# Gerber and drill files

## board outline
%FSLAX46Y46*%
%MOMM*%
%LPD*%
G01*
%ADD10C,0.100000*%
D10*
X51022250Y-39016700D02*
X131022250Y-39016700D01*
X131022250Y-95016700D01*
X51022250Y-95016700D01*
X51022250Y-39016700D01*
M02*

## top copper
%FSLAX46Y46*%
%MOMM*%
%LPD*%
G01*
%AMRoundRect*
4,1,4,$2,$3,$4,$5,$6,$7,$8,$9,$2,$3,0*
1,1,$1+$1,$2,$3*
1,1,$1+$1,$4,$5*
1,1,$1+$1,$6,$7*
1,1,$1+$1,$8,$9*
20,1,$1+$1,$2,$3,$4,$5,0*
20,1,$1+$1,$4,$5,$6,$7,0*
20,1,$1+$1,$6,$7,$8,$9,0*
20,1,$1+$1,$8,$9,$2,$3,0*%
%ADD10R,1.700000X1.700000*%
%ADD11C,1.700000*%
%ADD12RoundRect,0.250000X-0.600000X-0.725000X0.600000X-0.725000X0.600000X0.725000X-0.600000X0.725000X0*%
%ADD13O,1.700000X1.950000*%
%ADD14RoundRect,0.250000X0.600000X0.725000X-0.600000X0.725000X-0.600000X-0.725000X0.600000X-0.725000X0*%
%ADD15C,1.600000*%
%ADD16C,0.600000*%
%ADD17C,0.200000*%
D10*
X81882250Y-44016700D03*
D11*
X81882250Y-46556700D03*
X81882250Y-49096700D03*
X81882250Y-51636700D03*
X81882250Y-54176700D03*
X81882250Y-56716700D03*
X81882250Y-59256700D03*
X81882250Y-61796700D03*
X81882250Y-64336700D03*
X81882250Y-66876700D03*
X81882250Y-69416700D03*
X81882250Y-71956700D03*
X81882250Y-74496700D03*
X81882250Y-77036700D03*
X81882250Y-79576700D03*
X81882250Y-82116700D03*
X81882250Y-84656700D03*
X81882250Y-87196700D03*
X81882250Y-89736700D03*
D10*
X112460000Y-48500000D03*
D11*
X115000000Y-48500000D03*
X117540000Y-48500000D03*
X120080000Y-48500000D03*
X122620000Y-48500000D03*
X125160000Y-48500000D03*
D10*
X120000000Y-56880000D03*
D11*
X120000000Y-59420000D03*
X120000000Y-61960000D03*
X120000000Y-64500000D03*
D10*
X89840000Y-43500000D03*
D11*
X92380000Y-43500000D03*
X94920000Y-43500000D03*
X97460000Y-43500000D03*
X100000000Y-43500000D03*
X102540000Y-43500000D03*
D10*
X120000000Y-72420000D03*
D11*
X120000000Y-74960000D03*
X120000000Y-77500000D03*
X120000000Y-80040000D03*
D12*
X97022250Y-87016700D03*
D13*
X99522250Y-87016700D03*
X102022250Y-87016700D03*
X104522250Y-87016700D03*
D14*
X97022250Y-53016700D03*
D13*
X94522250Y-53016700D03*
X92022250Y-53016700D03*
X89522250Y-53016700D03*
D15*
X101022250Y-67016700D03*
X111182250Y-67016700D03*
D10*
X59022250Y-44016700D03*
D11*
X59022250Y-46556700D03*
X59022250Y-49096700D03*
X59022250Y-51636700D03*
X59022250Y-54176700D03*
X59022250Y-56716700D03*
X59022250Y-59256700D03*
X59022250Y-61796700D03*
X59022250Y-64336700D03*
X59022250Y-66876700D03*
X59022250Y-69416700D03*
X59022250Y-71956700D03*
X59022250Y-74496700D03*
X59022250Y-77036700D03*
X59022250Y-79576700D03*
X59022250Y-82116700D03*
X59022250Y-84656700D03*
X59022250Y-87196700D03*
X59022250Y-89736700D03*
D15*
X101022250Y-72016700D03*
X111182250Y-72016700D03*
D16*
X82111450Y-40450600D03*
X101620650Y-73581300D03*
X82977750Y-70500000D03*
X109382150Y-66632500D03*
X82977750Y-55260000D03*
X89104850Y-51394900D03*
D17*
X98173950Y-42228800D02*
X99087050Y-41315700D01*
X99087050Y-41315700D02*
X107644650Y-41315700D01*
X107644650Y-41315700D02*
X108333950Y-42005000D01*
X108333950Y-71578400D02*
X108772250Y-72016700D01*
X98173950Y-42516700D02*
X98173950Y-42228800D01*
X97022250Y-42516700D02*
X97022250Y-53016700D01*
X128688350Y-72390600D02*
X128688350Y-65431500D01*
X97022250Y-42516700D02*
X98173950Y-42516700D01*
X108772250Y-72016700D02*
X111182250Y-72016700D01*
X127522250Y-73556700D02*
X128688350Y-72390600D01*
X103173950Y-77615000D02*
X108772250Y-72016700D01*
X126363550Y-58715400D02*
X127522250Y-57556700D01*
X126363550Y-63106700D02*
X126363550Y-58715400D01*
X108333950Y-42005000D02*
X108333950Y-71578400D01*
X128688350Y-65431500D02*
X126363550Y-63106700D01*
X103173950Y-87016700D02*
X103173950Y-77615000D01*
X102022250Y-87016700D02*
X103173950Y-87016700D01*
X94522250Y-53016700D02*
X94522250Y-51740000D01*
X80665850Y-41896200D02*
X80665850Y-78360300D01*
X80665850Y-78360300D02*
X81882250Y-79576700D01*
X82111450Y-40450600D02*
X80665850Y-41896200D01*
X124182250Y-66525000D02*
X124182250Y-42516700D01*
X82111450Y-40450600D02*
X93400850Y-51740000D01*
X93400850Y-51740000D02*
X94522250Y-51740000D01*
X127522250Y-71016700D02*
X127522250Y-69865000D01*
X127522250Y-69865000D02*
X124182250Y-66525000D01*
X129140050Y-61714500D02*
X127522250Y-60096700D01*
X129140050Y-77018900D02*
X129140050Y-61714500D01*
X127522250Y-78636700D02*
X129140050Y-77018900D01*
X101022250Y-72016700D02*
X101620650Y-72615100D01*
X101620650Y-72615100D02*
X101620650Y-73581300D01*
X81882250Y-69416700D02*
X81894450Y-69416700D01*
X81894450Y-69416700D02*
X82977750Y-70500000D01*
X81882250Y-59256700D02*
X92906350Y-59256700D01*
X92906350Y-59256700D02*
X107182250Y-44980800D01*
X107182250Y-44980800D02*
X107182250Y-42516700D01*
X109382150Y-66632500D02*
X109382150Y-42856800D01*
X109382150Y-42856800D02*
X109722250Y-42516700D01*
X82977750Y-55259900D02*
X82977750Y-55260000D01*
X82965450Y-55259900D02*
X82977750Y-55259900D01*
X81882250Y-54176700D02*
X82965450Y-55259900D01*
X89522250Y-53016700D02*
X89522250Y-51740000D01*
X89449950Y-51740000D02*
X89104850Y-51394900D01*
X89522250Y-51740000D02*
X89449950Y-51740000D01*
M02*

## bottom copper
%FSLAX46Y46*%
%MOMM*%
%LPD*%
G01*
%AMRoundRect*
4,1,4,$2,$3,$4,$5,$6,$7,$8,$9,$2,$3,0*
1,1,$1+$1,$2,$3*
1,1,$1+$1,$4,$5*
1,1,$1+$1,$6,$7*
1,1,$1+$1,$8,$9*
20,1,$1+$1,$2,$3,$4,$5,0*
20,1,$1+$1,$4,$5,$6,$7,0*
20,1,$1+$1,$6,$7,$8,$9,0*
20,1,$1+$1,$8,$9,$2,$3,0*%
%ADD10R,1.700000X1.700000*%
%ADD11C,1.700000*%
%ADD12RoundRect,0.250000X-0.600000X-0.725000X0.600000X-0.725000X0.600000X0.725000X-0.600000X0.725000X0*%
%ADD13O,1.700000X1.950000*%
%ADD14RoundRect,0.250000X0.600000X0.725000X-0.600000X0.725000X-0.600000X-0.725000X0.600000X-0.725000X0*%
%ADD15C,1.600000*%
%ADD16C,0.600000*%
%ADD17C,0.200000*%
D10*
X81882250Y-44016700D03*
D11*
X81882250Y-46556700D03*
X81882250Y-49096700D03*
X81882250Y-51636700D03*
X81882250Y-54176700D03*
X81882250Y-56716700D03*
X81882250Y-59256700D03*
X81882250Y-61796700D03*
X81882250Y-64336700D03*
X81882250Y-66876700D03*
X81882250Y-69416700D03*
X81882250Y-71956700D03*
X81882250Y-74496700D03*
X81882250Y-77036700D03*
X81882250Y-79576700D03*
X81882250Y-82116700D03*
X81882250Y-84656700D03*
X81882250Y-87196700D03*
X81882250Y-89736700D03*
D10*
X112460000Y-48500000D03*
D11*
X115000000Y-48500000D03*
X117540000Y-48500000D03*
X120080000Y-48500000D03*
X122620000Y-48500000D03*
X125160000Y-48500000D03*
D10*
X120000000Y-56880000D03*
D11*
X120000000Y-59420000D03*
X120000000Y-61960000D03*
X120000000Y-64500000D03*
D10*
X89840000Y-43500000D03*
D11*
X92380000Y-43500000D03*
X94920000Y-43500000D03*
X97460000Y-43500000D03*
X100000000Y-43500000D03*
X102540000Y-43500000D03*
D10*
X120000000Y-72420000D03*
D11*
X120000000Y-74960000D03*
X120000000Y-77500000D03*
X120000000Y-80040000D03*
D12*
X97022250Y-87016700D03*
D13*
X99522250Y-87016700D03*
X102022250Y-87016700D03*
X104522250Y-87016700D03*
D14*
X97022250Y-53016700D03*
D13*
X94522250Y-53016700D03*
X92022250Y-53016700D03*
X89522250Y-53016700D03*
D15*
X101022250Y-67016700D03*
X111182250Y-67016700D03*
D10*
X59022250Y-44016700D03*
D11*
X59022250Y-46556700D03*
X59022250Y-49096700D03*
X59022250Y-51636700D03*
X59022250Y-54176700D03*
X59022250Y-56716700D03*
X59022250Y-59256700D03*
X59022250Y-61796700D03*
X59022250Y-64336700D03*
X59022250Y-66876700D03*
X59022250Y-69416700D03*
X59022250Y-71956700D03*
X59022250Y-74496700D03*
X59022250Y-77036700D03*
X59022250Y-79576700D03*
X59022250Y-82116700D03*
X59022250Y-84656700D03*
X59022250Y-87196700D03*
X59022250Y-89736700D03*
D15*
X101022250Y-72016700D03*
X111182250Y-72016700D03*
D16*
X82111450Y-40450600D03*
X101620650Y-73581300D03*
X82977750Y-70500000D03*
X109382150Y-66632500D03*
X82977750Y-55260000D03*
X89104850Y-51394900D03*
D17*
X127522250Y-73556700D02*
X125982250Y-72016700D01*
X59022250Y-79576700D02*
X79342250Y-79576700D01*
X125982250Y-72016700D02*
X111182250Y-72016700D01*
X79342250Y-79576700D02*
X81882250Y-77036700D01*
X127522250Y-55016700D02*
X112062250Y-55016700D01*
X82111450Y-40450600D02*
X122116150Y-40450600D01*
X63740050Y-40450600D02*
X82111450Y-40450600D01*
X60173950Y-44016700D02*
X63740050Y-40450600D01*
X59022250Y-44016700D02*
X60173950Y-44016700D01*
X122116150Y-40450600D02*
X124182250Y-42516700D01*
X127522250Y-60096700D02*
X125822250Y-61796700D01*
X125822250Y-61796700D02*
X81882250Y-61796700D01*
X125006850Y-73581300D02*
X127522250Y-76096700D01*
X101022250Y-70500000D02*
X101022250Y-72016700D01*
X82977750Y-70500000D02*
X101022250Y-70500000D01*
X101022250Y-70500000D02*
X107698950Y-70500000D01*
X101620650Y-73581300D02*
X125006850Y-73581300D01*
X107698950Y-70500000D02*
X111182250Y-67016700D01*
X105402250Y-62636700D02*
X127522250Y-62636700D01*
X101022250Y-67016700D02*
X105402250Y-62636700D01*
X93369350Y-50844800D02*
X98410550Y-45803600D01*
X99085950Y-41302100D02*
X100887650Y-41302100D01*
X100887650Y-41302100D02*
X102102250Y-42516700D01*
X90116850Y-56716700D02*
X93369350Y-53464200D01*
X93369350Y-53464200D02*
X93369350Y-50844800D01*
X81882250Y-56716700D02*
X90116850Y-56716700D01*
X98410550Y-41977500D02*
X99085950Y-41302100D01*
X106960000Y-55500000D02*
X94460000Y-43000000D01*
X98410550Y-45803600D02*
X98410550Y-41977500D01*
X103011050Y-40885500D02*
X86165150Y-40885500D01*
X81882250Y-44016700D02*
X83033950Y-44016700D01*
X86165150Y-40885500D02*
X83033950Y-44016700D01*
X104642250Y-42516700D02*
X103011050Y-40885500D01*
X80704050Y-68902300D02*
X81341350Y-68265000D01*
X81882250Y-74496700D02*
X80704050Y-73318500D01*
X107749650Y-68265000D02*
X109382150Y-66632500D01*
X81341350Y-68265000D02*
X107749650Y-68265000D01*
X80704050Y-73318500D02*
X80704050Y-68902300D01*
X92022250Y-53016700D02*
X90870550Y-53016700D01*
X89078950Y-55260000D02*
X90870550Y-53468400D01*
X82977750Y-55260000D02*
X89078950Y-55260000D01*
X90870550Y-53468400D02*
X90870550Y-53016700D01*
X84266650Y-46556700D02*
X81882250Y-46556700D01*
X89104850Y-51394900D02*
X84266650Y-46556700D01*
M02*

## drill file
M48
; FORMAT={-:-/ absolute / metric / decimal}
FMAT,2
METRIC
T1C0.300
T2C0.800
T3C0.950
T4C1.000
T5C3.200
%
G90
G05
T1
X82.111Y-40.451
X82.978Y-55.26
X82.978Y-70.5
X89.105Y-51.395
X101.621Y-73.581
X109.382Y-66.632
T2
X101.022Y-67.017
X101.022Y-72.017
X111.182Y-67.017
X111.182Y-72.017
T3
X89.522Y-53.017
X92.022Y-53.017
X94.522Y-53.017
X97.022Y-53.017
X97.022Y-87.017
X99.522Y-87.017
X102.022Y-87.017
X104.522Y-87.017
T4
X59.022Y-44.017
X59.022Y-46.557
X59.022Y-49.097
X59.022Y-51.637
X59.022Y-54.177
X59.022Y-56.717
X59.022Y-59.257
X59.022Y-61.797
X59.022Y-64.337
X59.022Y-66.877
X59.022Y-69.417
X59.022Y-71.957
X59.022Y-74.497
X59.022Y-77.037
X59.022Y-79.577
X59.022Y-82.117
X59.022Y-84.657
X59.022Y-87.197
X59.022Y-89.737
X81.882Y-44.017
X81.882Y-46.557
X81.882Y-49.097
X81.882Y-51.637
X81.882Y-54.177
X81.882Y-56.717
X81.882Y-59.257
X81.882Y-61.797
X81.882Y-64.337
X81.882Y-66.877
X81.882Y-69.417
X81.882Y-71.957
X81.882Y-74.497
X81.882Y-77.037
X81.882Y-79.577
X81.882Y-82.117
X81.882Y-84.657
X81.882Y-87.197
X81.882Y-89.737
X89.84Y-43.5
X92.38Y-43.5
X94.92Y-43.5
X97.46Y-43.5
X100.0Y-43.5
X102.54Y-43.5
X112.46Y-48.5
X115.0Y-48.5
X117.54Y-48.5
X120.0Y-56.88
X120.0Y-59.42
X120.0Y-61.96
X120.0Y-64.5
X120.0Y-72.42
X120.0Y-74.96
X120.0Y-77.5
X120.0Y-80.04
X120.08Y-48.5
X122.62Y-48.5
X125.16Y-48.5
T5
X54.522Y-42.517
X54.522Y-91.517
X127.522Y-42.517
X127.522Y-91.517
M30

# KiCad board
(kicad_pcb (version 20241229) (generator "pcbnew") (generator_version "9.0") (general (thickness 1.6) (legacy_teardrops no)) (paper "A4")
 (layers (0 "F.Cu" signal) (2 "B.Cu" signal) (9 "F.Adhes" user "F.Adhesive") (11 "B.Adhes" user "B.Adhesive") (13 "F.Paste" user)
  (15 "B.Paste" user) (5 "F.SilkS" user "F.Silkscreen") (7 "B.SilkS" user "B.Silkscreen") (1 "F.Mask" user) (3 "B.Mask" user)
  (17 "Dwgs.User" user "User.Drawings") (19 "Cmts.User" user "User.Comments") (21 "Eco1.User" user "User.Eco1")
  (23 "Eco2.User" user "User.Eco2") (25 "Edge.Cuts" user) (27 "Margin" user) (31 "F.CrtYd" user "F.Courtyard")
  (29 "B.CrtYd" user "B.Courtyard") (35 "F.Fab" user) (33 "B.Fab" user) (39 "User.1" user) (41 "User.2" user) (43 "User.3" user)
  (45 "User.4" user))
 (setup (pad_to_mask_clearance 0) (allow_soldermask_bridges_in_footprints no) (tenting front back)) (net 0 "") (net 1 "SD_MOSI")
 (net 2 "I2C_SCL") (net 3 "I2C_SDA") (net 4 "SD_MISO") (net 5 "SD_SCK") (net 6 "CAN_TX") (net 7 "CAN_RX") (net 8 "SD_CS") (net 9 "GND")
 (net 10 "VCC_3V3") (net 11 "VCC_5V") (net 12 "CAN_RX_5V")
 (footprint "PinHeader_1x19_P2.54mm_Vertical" (layer "F.Cu") (at 81.88225 44.0167)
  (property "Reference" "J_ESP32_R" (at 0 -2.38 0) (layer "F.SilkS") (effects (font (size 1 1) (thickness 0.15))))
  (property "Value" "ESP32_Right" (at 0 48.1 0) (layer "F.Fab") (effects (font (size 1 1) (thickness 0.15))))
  (pad "1" thru_hole rect (at 0 0) (size 1.7 1.7) (drill 1) (layers "*.Cu" "*.Mask") (remove_unused_layers no) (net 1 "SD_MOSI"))
  (pad "2" thru_hole circle (at 0 2.54) (size 1.7 1.7) (drill 1) (layers "*.Cu" "*.Mask") (remove_unused_layers no) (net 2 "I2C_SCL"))
  (pad "3" thru_hole circle (at 0 5.08) (size 1.7 1.7) (drill 1) (layers "*.Cu" "*.Mask") (remove_unused_layers no))
  (pad "4" thru_hole circle (at 0 7.62) (size 1.7 1.7) (drill 1) (layers "*.Cu" "*.Mask") (remove_unused_layers no))
  (pad "5" thru_hole circle (at 0 10.16) (size 1.7 1.7) (drill 1) (layers "*.Cu" "*.Mask") (remove_unused_layers no) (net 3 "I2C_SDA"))
  (pad "6" thru_hole circle (at 0 12.7) (size 1.7 1.7) (drill 1) (layers "*.Cu" "*.Mask") (remove_unused_layers no) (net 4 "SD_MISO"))
  (pad "7" thru_hole circle (at 0 15.24) (size 1.7 1.7) (drill 1) (layers "*.Cu" "*.Mask") (remove_unused_layers no) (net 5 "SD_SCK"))
  (pad "8" thru_hole circle (at 0 17.78) (size 1.7 1.7) (drill 1) (layers "*.Cu" "*.Mask") (remove_unused_layers no) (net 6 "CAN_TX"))
  (pad "9" thru_hole circle (at 0 20.32) (size 1.7 1.7) (drill 1) (layers "*.Cu" "*.Mask") (remove_unused_layers no))
  (pad "10" thru_hole circle (at 0 22.86) (size 1.7 1.7) (drill 1) (layers "*.Cu" "*.Mask") (remove_unused_layers no))
  (pad "11" thru_hole circle (at 0 25.4) (size 1.7 1.7) (drill 1) (layers "*.Cu" "*.Mask") (remove_unused_layers no) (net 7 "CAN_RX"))
  (pad "12" thru_hole circle (at 0 27.94) (size 1.7 1.7) (drill 1) (layers "*.Cu" "*.Mask") (remove_unused_layers no))
  (pad "13" thru_hole circle (at 0 30.48) (size 1.7 1.7) (drill 1) (layers "*.Cu" "*.Mask") (remove_unused_layers no) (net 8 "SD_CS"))
  (pad "14" thru_hole circle (at 0 33.02) (size 1.7 1.7) (drill 1) (layers "*.Cu" "*.Mask") (remove_unused_layers no) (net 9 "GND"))
  (pad "15" thru_hole circle (at 0 35.56) (size 1.7 1.7) (drill 1) (layers "*.Cu" "*.Mask") (remove_unused_layers no) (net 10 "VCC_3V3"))
  (pad "16" thru_hole circle (at 0 38.1) (size 1.7 1.7) (drill 1) (layers "*.Cu" "*.Mask") (remove_unused_layers no))
  (pad "17" thru_hole circle (at 0 40.64) (size 1.7 1.7) (drill 1) (layers "*.Cu" "*.Mask") (remove_unused_layers no))
  (pad "18" thru_hole circle (at 0 43.18) (size 1.7 1.7) (drill 1) (layers "*.Cu" "*.Mask") (remove_unused_layers no))
  (pad "19" thru_hole circle (at 0 45.72) (size 1.7 1.7) (drill 1) (layers "*.Cu" "*.Mask") (remove_unused_layers no)))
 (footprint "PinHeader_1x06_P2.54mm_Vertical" (layer "F.Cu") (at 112.46 48.5 90)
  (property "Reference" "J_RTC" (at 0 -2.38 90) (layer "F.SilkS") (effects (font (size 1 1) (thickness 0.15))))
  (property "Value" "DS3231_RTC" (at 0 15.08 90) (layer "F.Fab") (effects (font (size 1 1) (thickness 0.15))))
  (pad "1" thru_hole rect (at 0 0 90) (size 1.7 1.7) (drill 1) (layers "*.Cu" "*.Mask") (remove_unused_layers no))
  (pad "2" thru_hole circle (at 0 2.54 90) (size 1.7 1.7) (drill 1) (layers "*.Cu" "*.Mask") (remove_unused_layers no))
  (pad "3" thru_hole circle (at 0 5.08 90) (size 1.7 1.7) (drill 1) (layers "*.Cu" "*.Mask") (remove_unused_layers no) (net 2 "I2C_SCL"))
  (pad "4" thru_hole circle (at 0 7.62 90) (size 1.7 1.7) (drill 1) (layers "*.Cu" "*.Mask") (remove_unused_layers no) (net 3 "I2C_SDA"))
  (pad "5" thru_hole circle (at 0 10.16 90) (size 1.7 1.7) (drill 1) (layers "*.Cu" "*.Mask") (remove_unused_layers no) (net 10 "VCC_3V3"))
  (pad "6" thru_hole circle (at 0 12.7 90) (size 1.7 1.7) (drill 1) (layers "*.Cu" "*.Mask") (remove_unused_layers no) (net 9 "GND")))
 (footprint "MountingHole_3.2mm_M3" (layer "F.Cu") (at 127.52225 91.5167)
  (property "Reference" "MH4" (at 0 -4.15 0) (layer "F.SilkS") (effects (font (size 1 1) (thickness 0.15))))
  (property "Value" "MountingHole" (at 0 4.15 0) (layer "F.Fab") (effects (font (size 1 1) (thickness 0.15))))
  (pad "" np_thru_hole circle (at 0 0) (size 3.2 3.2) (drill 3.2) (layers "*.Cu" "*.Mask")))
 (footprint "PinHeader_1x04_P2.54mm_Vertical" (layer "F.Cu") (at 120 56.88)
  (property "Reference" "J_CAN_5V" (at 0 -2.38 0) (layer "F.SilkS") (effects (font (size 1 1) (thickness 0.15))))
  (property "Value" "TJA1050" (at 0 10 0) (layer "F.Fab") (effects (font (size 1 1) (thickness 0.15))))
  (pad "1" thru_hole rect (at 0 0) (size 1.7 1.7) (drill 1) (layers "*.Cu" "*.Mask") (remove_unused_layers no) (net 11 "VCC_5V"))
  (pad "2" thru_hole circle (at 0 2.54) (size 1.7 1.7) (drill 1) (layers "*.Cu" "*.Mask") (remove_unused_layers no) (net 9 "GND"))
  (pad "3" thru_hole circle (at 0 5.08) (size 1.7 1.7) (drill 1) (layers "*.Cu" "*.Mask") (remove_unused_layers no) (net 6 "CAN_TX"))
  (pad "4" thru_hole circle (at 0 7.62) (size 1.7 1.7) (drill 1) (layers "*.Cu" "*.Mask") (remove_unused_layers no) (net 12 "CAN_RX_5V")))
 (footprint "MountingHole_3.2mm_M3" (layer "F.Cu") (at 54.52225 91.5167)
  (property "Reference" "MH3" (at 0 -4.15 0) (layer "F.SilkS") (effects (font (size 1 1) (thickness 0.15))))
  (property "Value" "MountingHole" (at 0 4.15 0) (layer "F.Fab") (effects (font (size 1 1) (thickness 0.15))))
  (pad "" np_thru_hole circle (at 0 0) (size 3.2 3.2) (drill 3.2) (layers "*.Cu" "*.Mask")))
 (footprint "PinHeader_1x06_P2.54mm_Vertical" (layer "F.Cu") (at 89.84 43.5 90)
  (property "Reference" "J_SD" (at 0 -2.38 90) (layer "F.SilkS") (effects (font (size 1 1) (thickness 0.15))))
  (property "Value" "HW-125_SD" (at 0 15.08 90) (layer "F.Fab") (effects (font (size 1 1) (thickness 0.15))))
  (pad "1" thru_hole rect (at 0 0 90) (size 1.7 1.7) (drill 1) (layers "*.Cu" "*.Mask") (remove_unused_layers no) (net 9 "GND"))
  (pad "2" thru_hole circle (at 0 2.54 90) (size 1.7 1.7) (drill 1) (layers "*.Cu" "*.Mask") (remove_unused_layers no) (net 11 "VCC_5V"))
  (pad "3" thru_hole circle (at 0 5.08 90) (size 1.7 1.7) (drill 1) (layers "*.Cu" "*.Mask") (remove_unused_layers no) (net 4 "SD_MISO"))
  (pad "4" thru_hole circle (at 0 7.62 90) (size 1.7 1.7) (drill 1) (layers "*.Cu" "*.Mask") (remove_unused_layers no) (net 1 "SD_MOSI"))
  (pad "5" thru_hole circle (at 0 10.16 90) (size 1.7 1.7) (drill 1) (layers "*.Cu" "*.Mask") (remove_unused_layers no) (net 5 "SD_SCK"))
  (pad "6" thru_hole circle (at 0 12.7 90) (size 1.7 1.7) (drill 1) (layers "*.Cu" "*.Mask") (remove_unused_layers no) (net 8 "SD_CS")))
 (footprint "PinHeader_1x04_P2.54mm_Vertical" (layer "F.Cu") (at 120 72.42)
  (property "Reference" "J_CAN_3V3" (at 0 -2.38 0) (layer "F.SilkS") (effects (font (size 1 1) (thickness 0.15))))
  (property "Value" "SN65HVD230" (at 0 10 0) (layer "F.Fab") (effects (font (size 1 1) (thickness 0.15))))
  (pad "1" thru_hole rect (at 0 0) (size 1.7 1.7) (drill 1) (layers "*.Cu" "*.Mask") (remove_unused_layers no) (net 10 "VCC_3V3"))
  (pad "2" thru_hole circle (at 0 2.54) (size 1.7 1.7) (drill 1) (layers "*.Cu" "*.Mask") (remove_unused_layers no) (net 9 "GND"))
  (pad "3" thru_hole circle (at 0 5.08) (size 1.7 1.7) (drill 1) (layers "*.Cu" "*.Mask") (remove_unused_layers no) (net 7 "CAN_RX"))
  (pad "4" thru_hole circle (at 0 7.62) (size 1.7 1.7) (drill 1) (layers "*.Cu" "*.Mask") (remove_unused_layers no) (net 6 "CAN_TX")))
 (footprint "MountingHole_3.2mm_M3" (layer "F.Cu") (at 127.52225 42.5167)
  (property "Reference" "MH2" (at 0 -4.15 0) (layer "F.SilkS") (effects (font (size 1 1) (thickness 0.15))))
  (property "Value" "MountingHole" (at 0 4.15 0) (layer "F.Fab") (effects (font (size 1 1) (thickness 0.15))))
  (pad "" np_thru_hole circle (at 0 0) (size 3.2 3.2) (drill 3.2) (layers "*.Cu" "*.Mask")))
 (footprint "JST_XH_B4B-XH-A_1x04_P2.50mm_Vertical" (layer "F.Cu") (at 97.02225 87.0167)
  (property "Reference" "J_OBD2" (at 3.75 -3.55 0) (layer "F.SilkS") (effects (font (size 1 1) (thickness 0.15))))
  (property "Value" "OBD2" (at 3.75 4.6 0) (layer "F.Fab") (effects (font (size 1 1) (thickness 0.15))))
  (pad "1" thru_hole roundrect (at 0 0) (size 1.7 1.95) (drill 0.95) (layers "*.Cu" "*.Mask") (remove_unused_layers no)
   (roundrect_rratio 0.147059))
  (pad "2" thru_hole oval (at 2.5 0) (size 1.7 1.95) (drill 0.95) (layers "*.Cu" "*.Mask") (remove_unused_layers no))
  (pad "3" thru_hole oval (at 5 0) (size 1.7 1.95) (drill 0.95) (layers "*.Cu" "*.Mask") (remove_unused_layers no) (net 9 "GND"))
  (pad "4" thru_hole oval (at 7.5 0) (size 1.7 1.95) (drill 0.95) (layers "*.Cu" "*.Mask") (remove_unused_layers no)))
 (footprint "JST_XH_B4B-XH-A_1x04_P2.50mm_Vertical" (layer "F.Cu") (at 97.02225 53.0167 180)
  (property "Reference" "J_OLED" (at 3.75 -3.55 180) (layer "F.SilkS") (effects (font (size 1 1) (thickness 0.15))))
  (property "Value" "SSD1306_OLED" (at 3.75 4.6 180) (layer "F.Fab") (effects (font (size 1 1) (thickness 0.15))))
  (pad "1" thru_hole roundrect (at 0 0 180) (size 1.7 1.95) (drill 0.95) (layers "*.Cu" "*.Mask") (remove_unused_layers no)
   (roundrect_rratio 0.147059) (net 9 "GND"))
  (pad "2" thru_hole oval (at 2.5 0 180) (size 1.7 1.95) (drill 0.95) (layers "*.Cu" "*.Mask") (remove_unused_layers no) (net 10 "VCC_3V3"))
  (pad "3" thru_hole oval (at 5 0 180) (size 1.7 1.95) (drill 0.95) (layers "*.Cu" "*.Mask") (remove_unused_layers no) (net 3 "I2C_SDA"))
  (pad "4" thru_hole oval (at 7.5 0 180) (size 1.7 1.95) (drill 0.95) (layers "*.Cu" "*.Mask") (remove_unused_layers no) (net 2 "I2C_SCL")))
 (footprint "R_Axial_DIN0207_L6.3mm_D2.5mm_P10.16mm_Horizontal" (layer "F.Cu") (at 101.02225 67.0167)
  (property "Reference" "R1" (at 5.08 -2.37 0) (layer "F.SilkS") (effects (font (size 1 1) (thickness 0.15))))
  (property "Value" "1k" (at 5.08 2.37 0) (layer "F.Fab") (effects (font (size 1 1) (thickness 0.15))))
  (pad "1" thru_hole circle (at 0 0) (size 1.6 1.6) (drill 0.8) (layers "*.Cu" "*.Mask") (remove_unused_layers no) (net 12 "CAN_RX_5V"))
  (pad "2" thru_hole circle (at 10.16 0) (size 1.6 1.6) (drill 0.8) (layers "*.Cu" "*.Mask") (remove_unused_layers no) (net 7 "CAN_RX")))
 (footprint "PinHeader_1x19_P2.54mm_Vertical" (layer "F.Cu") (at 59.02225 44.0167)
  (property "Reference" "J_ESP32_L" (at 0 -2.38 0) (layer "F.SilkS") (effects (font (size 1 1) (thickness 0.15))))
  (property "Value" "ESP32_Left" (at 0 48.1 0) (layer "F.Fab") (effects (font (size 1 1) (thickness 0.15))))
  (pad "1" thru_hole rect (at 0 0) (size 1.7 1.7) (drill 1) (layers "*.Cu" "*.Mask") (remove_unused_layers no) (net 10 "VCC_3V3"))
  (pad "2" thru_hole circle (at 0 2.54) (size 1.7 1.7) (drill 1) (layers "*.Cu" "*.Mask") (remove_unused_layers no))
  (pad "3" thru_hole circle (at 0 5.08) (size 1.7 1.7) (drill 1) (layers "*.Cu" "*.Mask") (remove_unused_layers no))
  (pad "4" thru_hole circle (at 0 7.62) (size 1.7 1.7) (drill 1) (layers "*.Cu" "*.Mask") (remove_unused_layers no))
  (pad "5" thru_hole circle (at 0 10.16) (size 1.7 1.7) (drill 1) (layers "*.Cu" "*.Mask") (remove_unused_layers no))
  (pad "6" thru_hole circle (at 0 12.7) (size 1.7 1.7) (drill 1) (layers "*.Cu" "*.Mask") (remove_unused_layers no))
  (pad "7" thru_hole circle (at 0 15.24) (size 1.7 1.7) (drill 1) (layers "*.Cu" "*.Mask") (remove_unused_layers no))
  (pad "8" thru_hole circle (at 0 17.78) (size 1.7 1.7) (drill 1) (layers "*.Cu" "*.Mask") (remove_unused_layers no))
  (pad "9" thru_hole circle (at 0 20.32) (size 1.7 1.7) (drill 1) (layers "*.Cu" "*.Mask") (remove_unused_layers no))
  (pad "10" thru_hole circle (at 0 22.86) (size 1.7 1.7) (drill 1) (layers "*.Cu" "*.Mask") (remove_unused_layers no))
  (pad "11" thru_hole circle (at 0 25.4) (size 1.7 1.7) (drill 1) (layers "*.Cu" "*.Mask") (remove_unused_layers no))
  (pad "12" thru_hole circle (at 0 27.94) (size 1.7 1.7) (drill 1) (layers "*.Cu" "*.Mask") (remove_unused_layers no))
  (pad "13" thru_hole circle (at 0 30.48) (size 1.7 1.7) (drill 1) (layers "*.Cu" "*.Mask") (remove_unused_layers no))
  (pad "14" thru_hole circle (at 0 33.02) (size 1.7 1.7) (drill 1) (layers "*.Cu" "*.Mask") (remove_unused_layers no))
  (pad "15" thru_hole circle (at 0 35.56) (size 1.7 1.7) (drill 1) (layers "*.Cu" "*.Mask") (remove_unused_layers no) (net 9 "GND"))
  (pad "16" thru_hole circle (at 0 38.1) (size 1.7 1.7) (drill 1) (layers "*.Cu" "*.Mask") (remove_unused_layers no) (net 11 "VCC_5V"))
  (pad "17" thru_hole circle (at 0 40.64) (size 1.7 1.7) (drill 1) (layers "*.Cu" "*.Mask") (remove_unused_layers no))
  (pad "18" thru_hole circle (at 0 43.18) (size 1.7 1.7) (drill 1) (layers "*.Cu" "*.Mask") (remove_unused_layers no))
  (pad "19" thru_hole circle (at 0 45.72) (size 1.7 1.7) (drill 1) (layers "*.Cu" "*.Mask") (remove_unused_layers no)))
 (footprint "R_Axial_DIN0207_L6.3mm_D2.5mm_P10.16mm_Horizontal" (layer "F.Cu") (at 101.02225 72.0167)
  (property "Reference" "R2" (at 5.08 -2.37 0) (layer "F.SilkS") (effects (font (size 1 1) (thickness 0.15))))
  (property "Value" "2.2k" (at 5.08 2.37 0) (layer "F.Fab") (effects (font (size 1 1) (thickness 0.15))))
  (pad "1" thru_hole circle (at 0 0) (size 1.6 1.6) (drill 0.8) (layers "*.Cu" "*.Mask") (remove_unused_layers no) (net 7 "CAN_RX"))
  (pad "2" thru_hole circle (at 10.16 0) (size 1.6 1.6) (drill 0.8) (layers "*.Cu" "*.Mask") (remove_unused_layers no) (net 9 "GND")))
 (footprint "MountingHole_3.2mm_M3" (layer "F.Cu") (at 54.52225 42.5167)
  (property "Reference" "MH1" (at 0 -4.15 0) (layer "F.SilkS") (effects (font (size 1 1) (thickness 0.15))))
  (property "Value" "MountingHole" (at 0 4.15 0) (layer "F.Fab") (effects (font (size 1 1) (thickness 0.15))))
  (pad "" np_thru_hole circle (at 0 0) (size 3.2 3.2) (drill 3.2) (layers "*.Cu" "*.Mask")))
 (gr_rect (start 51.02225 39.0167) (end 131.02225 95.0167) (stroke (width 0.1) (type default)) (fill no) (layer "Edge.Cuts"))
 (segment (start 98.17395 42.2288) (end 99.08705 41.3157) (width 0.2) (layer "F.Cu") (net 9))
 (segment (start 99.08705 41.3157) (end 107.64465 41.3157) (width 0.2) (layer "F.Cu") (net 9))
 (segment (start 107.64465 41.3157) (end 108.33395 42.005) (width 0.2) (layer "F.Cu") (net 9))
 (segment (start 108.33395 71.5784) (end 108.77225 72.0167) (width 0.2) (layer "F.Cu") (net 9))
 (segment (start 98.17395 42.5167) (end 98.17395 42.2288) (width 0.2) (layer "F.Cu") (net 9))
 (segment (start 97.02225 42.5167) (end 97.02225 53.0167) (width 0.2) (layer "F.Cu") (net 9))
 (segment (start 128.68835 72.3906) (end 128.68835 65.4315) (width 0.2) (layer "F.Cu") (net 9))
 (segment (start 97.02225 42.5167) (end 98.17395 42.5167) (width 0.2) (layer "F.Cu") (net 9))
 (segment (start 108.77225 72.0167) (end 111.18225 72.0167) (width 0.2) (layer "F.Cu") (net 9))
 (segment (start 127.52225 73.5567) (end 128.68835 72.3906) (width 0.2) (layer "F.Cu") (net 9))
 (segment (start 103.17395 77.615) (end 108.77225 72.0167) (width 0.2) (layer "F.Cu") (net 9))
 (segment (start 126.36355 58.7154) (end 127.52225 57.5567) (width 0.2) (layer "F.Cu") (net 9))
 (segment (start 126.36355 63.1067) (end 126.36355 58.7154) (width 0.2) (layer "F.Cu") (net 9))
 (segment (start 108.33395 42.005) (end 108.33395 71.5784) (width 0.2) (layer "F.Cu") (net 9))
 (segment (start 128.68835 65.4315) (end 126.36355 63.1067) (width 0.2) (layer "F.Cu") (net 9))
 (segment (start 103.17395 87.0167) (end 103.17395 77.615) (width 0.2) (layer "F.Cu") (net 9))
 (segment (start 102.02225 87.0167) (end 103.17395 87.0167) (width 0.2) (layer "F.Cu") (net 9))
 (segment (start 127.52225 73.5567) (end 125.98225 72.0167) (width 0.2) (layer "B.Cu") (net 9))
 (segment (start 59.02225 79.5767) (end 79.34225 79.5767) (width 0.2) (layer "B.Cu") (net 9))
 (segment (start 125.98225 72.0167) (end 111.18225 72.0167) (width 0.2) (layer "B.Cu") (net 9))
 (segment (start 79.34225 79.5767) (end 81.88225 77.0367) (width 0.2) (layer "B.Cu") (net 9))
 (segment (start 127.52225 55.0167) (end 112.06225 55.0167) (width 0.2) (layer "B.Cu") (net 11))
 (segment (start 94.52225 53.0167) (end 94.52225 51.74) (width 0.2) (layer "F.Cu") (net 10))
 (segment (start 80.66585 41.8962) (end 80.66585 78.3603) (width 0.2) (layer "F.Cu") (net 10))
 (segment (start 80.66585 78.3603) (end 81.88225 79.5767) (width 0.2) (layer "F.Cu") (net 10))
 (segment (start 82.11145 40.4506) (end 80.66585 41.8962) (width 0.2) (layer "F.Cu") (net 10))
 (segment (start 124.18225 66.525) (end 124.18225 42.5167) (width 0.2) (layer "F.Cu") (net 10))
 (segment (start 82.11145 40.4506) (end 93.40085 51.74) (width 0.2) (layer "F.Cu") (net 10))
 (segment (start 93.40085 51.74) (end 94.52225 51.74) (width 0.2) (layer "F.Cu") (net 10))
 (segment (start 127.52225 71.0167) (end 127.52225 69.865) (width 0.2) (layer "F.Cu") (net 10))
 (segment (start 127.52225 69.865) (end 124.18225 66.525) (width 0.2) (layer "F.Cu") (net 10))
 (via (at 82.11145 40.4506) (size 0.6) (drill 0.3) (layers "F.Cu" "B.Cu") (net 10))
 (segment (start 82.11145 40.4506) (end 122.11615 40.4506) (width 0.2) (layer "B.Cu") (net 10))
 (segment (start 63.74005 40.4506) (end 82.11145 40.4506) (width 0.2) (layer "B.Cu") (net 10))
 (segment (start 60.17395 44.0167) (end 63.74005 40.4506) (width 0.2) (layer "B.Cu") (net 10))
 (segment (start 59.02225 44.0167) (end 60.17395 44.0167) (width 0.2) (layer "B.Cu") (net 10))
 (segment (start 122.11615 40.4506) (end 124.18225 42.5167) (width 0.2) (layer "B.Cu") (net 10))
 (segment (start 129.14005 61.7145) (end 127.52225 60.0967) (width 0.2) (layer "F.Cu") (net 6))
 (segment (start 129.14005 77.0189) (end 129.14005 61.7145) (width 0.2) (layer "F.Cu") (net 6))
 (segment (start 127.52225 78.6367) (end 129.14005 77.0189) (width 0.2) (layer "F.Cu") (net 6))
 (segment (start 127.52225 60.0967) (end 125.82225 61.7967) (width 0.2) (layer "B.Cu") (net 6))
 (segment (start 125.82225 61.7967) (end 81.88225 61.7967) (width 0.2) (layer "B.Cu") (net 6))
 (segment (start 101.02225 72.0167) (end 101.62065 72.6151) (width 0.2) (layer "F.Cu") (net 7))
 (segment (start 101.62065 72.6151) (end 101.62065 73.5813) (width 0.2) (layer "F.Cu") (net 7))
 (segment (start 81.88225 69.4167) (end 81.89445 69.4167) (width 0.2) (layer "F.Cu") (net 7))
 (segment (start 81.89445 69.4167) (end 82.97775 70.5) (width 0.2) (layer "F.Cu") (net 7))
 (via (at 101.62065 73.5813) (size 0.6) (drill 0.3) (layers "F.Cu" "B.Cu") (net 7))
 (via (at 82.97775 70.5) (size 0.6) (drill 0.3) (layers "F.Cu" "B.Cu") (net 7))
 (segment (start 125.00685 73.5813) (end 127.52225 76.0967) (width 0.2) (layer "B.Cu") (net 7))
 (segment (start 101.02225 70.5) (end 101.02225 72.0167) (width 0.2) (layer "B.Cu") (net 7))
 (segment (start 82.97775 70.5) (end 101.02225 70.5) (width 0.2) (layer "B.Cu") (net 7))
 (segment (start 101.02225 70.5) (end 107.69895 70.5) (width 0.2) (layer "B.Cu") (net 7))
 (segment (start 101.62065 73.5813) (end 125.00685 73.5813) (width 0.2) (layer "B.Cu") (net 7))
 (segment (start 107.69895 70.5) (end 111.18225 67.0167) (width 0.2) (layer "B.Cu") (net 7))
 (segment (start 105.40225 62.6367) (end 127.52225 62.6367) (width 0.2) (layer "B.Cu") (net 12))
 (segment (start 101.02225 67.0167) (end 105.40225 62.6367) (width 0.2) (layer "B.Cu") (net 12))
 (segment (start 93.36935 50.8448) (end 98.41055 45.8036) (width 0.2) (layer "B.Cu") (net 4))
 (segment (start 99.08595 41.3021) (end 100.88765 41.3021) (width 0.2) (layer "B.Cu") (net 4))
 (segment (start 100.88765 41.3021) (end 102.10225 42.5167) (width 0.2) (layer "B.Cu") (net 4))
 (segment (start 90.11685 56.7167) (end 93.36935 53.4642) (width 0.2) (layer "B.Cu") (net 4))
 (segment (start 93.36935 53.4642) (end 93.36935 50.8448) (width 0.2) (layer "B.Cu") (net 4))
 (segment (start 81.88225 56.7167) (end 90.11685 56.7167) (width 0.2) (layer "B.Cu") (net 4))
 (segment (start 98.41055 41.9775) (end 99.08595 41.3021) (width 0.2) (layer "B.Cu") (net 4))
 (segment (start 106.96 55.5) (end 94.46 43) (width 0.2) (layer "B.Cu") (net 4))
 (segment (start 98.41055 45.8036) (end 98.41055 41.9775) (width 0.2) (layer "B.Cu") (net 4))
 (segment (start 103.01105 40.8855) (end 86.16515 40.8855) (width 0.2) (layer "B.Cu") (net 1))
 (segment (start 81.88225 44.0167) (end 83.03395 44.0167) (width 0.2) (layer "B.Cu") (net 1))
 (segment (start 86.16515 40.8855) (end 83.03395 44.0167) (width 0.2) (layer "B.Cu") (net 1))
 (segment (start 104.64225 42.5167) (end 103.01105 40.8855) (width 0.2) (layer "B.Cu") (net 1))
 (segment (start 81.88225 59.2567) (end 92.90635 59.2567) (width 0.2) (layer "F.Cu") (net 5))
 (segment (start 92.90635 59.2567) (end 107.18225 44.9808) (width 0.2) (layer "F.Cu") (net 5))
 (segment (start 107.18225 44.9808) (end 107.18225 42.5167) (width 0.2) (layer "F.Cu") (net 5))
 (segment (start 109.38215 66.6325) (end 109.38215 42.8568) (width 0.2) (layer "F.Cu") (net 8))
 (segment (start 109.38215 42.8568) (end 109.72225 42.5167) (width 0.2) (layer "F.Cu") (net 8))
 (via (at 109.38215 66.6325) (size 0.6) (drill 0.3) (layers "F.Cu" "B.Cu") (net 8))
 (segment (start 80.70405 68.9023) (end 81.34135 68.265) (width 0.2) (layer "B.Cu") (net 8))
 (segment (start 81.88225 74.4967) (end 80.70405 73.3185) (width 0.2) (layer "B.Cu") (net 8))
 (segment (start 107.74965 68.265) (end 109.38215 66.6325) (width 0.2) (layer "B.Cu") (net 8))
 (segment (start 81.34135 68.265) (end 107.74965 68.265) (width 0.2) (layer "B.Cu") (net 8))
 (segment (start 80.70405 73.3185) (end 80.70405 68.9023) (width 0.2) (layer "B.Cu") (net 8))
 (segment (start 82.97775 55.2599) (end 82.97775 55.26) (width 0.2) (layer "F.Cu") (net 3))
 (segment (start 82.96545 55.2599) (end 82.97775 55.2599) (width 0.2) (layer "F.Cu") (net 3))
 (segment (start 81.88225 54.1767) (end 82.96545 55.2599) (width 0.2) (layer "F.Cu") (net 3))
 (via (at 82.97775 55.26) (size 0.6) (drill 0.3) (layers "F.Cu" "B.Cu") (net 3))
 (segment (start 92.02225 53.0167) (end 90.87055 53.0167) (width 0.2) (layer "B.Cu") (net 3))
 (segment (start 89.07895 55.26) (end 90.87055 53.4684) (width 0.2) (layer "B.Cu") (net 3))
 (segment (start 82.97775 55.26) (end 89.07895 55.26) (width 0.2) (layer "B.Cu") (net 3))
 (segment (start 90.87055 53.4684) (end 90.87055 53.0167) (width 0.2) (layer "B.Cu") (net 3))
 (segment (start 89.52225 53.0167) (end 89.52225 51.74) (width 0.2) (layer "F.Cu") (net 2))
 (segment (start 89.44995 51.74) (end 89.10485 51.3949) (width 0.2) (layer "F.Cu") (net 2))
 (segment (start 89.52225 51.74) (end 89.44995 51.74) (width 0.2) (layer "F.Cu") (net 2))
 (via (at 89.10485 51.3949) (size 0.6) (drill 0.3) (layers "F.Cu" "B.Cu") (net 2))
 (segment (start 84.26665 46.5567) (end 81.88225 46.5567) (width 0.2) (layer "B.Cu") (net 2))
 (segment (start 89.10485 51.3949) (end 84.26665 46.5567) (width 0.2) (layer "B.Cu") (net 2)))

